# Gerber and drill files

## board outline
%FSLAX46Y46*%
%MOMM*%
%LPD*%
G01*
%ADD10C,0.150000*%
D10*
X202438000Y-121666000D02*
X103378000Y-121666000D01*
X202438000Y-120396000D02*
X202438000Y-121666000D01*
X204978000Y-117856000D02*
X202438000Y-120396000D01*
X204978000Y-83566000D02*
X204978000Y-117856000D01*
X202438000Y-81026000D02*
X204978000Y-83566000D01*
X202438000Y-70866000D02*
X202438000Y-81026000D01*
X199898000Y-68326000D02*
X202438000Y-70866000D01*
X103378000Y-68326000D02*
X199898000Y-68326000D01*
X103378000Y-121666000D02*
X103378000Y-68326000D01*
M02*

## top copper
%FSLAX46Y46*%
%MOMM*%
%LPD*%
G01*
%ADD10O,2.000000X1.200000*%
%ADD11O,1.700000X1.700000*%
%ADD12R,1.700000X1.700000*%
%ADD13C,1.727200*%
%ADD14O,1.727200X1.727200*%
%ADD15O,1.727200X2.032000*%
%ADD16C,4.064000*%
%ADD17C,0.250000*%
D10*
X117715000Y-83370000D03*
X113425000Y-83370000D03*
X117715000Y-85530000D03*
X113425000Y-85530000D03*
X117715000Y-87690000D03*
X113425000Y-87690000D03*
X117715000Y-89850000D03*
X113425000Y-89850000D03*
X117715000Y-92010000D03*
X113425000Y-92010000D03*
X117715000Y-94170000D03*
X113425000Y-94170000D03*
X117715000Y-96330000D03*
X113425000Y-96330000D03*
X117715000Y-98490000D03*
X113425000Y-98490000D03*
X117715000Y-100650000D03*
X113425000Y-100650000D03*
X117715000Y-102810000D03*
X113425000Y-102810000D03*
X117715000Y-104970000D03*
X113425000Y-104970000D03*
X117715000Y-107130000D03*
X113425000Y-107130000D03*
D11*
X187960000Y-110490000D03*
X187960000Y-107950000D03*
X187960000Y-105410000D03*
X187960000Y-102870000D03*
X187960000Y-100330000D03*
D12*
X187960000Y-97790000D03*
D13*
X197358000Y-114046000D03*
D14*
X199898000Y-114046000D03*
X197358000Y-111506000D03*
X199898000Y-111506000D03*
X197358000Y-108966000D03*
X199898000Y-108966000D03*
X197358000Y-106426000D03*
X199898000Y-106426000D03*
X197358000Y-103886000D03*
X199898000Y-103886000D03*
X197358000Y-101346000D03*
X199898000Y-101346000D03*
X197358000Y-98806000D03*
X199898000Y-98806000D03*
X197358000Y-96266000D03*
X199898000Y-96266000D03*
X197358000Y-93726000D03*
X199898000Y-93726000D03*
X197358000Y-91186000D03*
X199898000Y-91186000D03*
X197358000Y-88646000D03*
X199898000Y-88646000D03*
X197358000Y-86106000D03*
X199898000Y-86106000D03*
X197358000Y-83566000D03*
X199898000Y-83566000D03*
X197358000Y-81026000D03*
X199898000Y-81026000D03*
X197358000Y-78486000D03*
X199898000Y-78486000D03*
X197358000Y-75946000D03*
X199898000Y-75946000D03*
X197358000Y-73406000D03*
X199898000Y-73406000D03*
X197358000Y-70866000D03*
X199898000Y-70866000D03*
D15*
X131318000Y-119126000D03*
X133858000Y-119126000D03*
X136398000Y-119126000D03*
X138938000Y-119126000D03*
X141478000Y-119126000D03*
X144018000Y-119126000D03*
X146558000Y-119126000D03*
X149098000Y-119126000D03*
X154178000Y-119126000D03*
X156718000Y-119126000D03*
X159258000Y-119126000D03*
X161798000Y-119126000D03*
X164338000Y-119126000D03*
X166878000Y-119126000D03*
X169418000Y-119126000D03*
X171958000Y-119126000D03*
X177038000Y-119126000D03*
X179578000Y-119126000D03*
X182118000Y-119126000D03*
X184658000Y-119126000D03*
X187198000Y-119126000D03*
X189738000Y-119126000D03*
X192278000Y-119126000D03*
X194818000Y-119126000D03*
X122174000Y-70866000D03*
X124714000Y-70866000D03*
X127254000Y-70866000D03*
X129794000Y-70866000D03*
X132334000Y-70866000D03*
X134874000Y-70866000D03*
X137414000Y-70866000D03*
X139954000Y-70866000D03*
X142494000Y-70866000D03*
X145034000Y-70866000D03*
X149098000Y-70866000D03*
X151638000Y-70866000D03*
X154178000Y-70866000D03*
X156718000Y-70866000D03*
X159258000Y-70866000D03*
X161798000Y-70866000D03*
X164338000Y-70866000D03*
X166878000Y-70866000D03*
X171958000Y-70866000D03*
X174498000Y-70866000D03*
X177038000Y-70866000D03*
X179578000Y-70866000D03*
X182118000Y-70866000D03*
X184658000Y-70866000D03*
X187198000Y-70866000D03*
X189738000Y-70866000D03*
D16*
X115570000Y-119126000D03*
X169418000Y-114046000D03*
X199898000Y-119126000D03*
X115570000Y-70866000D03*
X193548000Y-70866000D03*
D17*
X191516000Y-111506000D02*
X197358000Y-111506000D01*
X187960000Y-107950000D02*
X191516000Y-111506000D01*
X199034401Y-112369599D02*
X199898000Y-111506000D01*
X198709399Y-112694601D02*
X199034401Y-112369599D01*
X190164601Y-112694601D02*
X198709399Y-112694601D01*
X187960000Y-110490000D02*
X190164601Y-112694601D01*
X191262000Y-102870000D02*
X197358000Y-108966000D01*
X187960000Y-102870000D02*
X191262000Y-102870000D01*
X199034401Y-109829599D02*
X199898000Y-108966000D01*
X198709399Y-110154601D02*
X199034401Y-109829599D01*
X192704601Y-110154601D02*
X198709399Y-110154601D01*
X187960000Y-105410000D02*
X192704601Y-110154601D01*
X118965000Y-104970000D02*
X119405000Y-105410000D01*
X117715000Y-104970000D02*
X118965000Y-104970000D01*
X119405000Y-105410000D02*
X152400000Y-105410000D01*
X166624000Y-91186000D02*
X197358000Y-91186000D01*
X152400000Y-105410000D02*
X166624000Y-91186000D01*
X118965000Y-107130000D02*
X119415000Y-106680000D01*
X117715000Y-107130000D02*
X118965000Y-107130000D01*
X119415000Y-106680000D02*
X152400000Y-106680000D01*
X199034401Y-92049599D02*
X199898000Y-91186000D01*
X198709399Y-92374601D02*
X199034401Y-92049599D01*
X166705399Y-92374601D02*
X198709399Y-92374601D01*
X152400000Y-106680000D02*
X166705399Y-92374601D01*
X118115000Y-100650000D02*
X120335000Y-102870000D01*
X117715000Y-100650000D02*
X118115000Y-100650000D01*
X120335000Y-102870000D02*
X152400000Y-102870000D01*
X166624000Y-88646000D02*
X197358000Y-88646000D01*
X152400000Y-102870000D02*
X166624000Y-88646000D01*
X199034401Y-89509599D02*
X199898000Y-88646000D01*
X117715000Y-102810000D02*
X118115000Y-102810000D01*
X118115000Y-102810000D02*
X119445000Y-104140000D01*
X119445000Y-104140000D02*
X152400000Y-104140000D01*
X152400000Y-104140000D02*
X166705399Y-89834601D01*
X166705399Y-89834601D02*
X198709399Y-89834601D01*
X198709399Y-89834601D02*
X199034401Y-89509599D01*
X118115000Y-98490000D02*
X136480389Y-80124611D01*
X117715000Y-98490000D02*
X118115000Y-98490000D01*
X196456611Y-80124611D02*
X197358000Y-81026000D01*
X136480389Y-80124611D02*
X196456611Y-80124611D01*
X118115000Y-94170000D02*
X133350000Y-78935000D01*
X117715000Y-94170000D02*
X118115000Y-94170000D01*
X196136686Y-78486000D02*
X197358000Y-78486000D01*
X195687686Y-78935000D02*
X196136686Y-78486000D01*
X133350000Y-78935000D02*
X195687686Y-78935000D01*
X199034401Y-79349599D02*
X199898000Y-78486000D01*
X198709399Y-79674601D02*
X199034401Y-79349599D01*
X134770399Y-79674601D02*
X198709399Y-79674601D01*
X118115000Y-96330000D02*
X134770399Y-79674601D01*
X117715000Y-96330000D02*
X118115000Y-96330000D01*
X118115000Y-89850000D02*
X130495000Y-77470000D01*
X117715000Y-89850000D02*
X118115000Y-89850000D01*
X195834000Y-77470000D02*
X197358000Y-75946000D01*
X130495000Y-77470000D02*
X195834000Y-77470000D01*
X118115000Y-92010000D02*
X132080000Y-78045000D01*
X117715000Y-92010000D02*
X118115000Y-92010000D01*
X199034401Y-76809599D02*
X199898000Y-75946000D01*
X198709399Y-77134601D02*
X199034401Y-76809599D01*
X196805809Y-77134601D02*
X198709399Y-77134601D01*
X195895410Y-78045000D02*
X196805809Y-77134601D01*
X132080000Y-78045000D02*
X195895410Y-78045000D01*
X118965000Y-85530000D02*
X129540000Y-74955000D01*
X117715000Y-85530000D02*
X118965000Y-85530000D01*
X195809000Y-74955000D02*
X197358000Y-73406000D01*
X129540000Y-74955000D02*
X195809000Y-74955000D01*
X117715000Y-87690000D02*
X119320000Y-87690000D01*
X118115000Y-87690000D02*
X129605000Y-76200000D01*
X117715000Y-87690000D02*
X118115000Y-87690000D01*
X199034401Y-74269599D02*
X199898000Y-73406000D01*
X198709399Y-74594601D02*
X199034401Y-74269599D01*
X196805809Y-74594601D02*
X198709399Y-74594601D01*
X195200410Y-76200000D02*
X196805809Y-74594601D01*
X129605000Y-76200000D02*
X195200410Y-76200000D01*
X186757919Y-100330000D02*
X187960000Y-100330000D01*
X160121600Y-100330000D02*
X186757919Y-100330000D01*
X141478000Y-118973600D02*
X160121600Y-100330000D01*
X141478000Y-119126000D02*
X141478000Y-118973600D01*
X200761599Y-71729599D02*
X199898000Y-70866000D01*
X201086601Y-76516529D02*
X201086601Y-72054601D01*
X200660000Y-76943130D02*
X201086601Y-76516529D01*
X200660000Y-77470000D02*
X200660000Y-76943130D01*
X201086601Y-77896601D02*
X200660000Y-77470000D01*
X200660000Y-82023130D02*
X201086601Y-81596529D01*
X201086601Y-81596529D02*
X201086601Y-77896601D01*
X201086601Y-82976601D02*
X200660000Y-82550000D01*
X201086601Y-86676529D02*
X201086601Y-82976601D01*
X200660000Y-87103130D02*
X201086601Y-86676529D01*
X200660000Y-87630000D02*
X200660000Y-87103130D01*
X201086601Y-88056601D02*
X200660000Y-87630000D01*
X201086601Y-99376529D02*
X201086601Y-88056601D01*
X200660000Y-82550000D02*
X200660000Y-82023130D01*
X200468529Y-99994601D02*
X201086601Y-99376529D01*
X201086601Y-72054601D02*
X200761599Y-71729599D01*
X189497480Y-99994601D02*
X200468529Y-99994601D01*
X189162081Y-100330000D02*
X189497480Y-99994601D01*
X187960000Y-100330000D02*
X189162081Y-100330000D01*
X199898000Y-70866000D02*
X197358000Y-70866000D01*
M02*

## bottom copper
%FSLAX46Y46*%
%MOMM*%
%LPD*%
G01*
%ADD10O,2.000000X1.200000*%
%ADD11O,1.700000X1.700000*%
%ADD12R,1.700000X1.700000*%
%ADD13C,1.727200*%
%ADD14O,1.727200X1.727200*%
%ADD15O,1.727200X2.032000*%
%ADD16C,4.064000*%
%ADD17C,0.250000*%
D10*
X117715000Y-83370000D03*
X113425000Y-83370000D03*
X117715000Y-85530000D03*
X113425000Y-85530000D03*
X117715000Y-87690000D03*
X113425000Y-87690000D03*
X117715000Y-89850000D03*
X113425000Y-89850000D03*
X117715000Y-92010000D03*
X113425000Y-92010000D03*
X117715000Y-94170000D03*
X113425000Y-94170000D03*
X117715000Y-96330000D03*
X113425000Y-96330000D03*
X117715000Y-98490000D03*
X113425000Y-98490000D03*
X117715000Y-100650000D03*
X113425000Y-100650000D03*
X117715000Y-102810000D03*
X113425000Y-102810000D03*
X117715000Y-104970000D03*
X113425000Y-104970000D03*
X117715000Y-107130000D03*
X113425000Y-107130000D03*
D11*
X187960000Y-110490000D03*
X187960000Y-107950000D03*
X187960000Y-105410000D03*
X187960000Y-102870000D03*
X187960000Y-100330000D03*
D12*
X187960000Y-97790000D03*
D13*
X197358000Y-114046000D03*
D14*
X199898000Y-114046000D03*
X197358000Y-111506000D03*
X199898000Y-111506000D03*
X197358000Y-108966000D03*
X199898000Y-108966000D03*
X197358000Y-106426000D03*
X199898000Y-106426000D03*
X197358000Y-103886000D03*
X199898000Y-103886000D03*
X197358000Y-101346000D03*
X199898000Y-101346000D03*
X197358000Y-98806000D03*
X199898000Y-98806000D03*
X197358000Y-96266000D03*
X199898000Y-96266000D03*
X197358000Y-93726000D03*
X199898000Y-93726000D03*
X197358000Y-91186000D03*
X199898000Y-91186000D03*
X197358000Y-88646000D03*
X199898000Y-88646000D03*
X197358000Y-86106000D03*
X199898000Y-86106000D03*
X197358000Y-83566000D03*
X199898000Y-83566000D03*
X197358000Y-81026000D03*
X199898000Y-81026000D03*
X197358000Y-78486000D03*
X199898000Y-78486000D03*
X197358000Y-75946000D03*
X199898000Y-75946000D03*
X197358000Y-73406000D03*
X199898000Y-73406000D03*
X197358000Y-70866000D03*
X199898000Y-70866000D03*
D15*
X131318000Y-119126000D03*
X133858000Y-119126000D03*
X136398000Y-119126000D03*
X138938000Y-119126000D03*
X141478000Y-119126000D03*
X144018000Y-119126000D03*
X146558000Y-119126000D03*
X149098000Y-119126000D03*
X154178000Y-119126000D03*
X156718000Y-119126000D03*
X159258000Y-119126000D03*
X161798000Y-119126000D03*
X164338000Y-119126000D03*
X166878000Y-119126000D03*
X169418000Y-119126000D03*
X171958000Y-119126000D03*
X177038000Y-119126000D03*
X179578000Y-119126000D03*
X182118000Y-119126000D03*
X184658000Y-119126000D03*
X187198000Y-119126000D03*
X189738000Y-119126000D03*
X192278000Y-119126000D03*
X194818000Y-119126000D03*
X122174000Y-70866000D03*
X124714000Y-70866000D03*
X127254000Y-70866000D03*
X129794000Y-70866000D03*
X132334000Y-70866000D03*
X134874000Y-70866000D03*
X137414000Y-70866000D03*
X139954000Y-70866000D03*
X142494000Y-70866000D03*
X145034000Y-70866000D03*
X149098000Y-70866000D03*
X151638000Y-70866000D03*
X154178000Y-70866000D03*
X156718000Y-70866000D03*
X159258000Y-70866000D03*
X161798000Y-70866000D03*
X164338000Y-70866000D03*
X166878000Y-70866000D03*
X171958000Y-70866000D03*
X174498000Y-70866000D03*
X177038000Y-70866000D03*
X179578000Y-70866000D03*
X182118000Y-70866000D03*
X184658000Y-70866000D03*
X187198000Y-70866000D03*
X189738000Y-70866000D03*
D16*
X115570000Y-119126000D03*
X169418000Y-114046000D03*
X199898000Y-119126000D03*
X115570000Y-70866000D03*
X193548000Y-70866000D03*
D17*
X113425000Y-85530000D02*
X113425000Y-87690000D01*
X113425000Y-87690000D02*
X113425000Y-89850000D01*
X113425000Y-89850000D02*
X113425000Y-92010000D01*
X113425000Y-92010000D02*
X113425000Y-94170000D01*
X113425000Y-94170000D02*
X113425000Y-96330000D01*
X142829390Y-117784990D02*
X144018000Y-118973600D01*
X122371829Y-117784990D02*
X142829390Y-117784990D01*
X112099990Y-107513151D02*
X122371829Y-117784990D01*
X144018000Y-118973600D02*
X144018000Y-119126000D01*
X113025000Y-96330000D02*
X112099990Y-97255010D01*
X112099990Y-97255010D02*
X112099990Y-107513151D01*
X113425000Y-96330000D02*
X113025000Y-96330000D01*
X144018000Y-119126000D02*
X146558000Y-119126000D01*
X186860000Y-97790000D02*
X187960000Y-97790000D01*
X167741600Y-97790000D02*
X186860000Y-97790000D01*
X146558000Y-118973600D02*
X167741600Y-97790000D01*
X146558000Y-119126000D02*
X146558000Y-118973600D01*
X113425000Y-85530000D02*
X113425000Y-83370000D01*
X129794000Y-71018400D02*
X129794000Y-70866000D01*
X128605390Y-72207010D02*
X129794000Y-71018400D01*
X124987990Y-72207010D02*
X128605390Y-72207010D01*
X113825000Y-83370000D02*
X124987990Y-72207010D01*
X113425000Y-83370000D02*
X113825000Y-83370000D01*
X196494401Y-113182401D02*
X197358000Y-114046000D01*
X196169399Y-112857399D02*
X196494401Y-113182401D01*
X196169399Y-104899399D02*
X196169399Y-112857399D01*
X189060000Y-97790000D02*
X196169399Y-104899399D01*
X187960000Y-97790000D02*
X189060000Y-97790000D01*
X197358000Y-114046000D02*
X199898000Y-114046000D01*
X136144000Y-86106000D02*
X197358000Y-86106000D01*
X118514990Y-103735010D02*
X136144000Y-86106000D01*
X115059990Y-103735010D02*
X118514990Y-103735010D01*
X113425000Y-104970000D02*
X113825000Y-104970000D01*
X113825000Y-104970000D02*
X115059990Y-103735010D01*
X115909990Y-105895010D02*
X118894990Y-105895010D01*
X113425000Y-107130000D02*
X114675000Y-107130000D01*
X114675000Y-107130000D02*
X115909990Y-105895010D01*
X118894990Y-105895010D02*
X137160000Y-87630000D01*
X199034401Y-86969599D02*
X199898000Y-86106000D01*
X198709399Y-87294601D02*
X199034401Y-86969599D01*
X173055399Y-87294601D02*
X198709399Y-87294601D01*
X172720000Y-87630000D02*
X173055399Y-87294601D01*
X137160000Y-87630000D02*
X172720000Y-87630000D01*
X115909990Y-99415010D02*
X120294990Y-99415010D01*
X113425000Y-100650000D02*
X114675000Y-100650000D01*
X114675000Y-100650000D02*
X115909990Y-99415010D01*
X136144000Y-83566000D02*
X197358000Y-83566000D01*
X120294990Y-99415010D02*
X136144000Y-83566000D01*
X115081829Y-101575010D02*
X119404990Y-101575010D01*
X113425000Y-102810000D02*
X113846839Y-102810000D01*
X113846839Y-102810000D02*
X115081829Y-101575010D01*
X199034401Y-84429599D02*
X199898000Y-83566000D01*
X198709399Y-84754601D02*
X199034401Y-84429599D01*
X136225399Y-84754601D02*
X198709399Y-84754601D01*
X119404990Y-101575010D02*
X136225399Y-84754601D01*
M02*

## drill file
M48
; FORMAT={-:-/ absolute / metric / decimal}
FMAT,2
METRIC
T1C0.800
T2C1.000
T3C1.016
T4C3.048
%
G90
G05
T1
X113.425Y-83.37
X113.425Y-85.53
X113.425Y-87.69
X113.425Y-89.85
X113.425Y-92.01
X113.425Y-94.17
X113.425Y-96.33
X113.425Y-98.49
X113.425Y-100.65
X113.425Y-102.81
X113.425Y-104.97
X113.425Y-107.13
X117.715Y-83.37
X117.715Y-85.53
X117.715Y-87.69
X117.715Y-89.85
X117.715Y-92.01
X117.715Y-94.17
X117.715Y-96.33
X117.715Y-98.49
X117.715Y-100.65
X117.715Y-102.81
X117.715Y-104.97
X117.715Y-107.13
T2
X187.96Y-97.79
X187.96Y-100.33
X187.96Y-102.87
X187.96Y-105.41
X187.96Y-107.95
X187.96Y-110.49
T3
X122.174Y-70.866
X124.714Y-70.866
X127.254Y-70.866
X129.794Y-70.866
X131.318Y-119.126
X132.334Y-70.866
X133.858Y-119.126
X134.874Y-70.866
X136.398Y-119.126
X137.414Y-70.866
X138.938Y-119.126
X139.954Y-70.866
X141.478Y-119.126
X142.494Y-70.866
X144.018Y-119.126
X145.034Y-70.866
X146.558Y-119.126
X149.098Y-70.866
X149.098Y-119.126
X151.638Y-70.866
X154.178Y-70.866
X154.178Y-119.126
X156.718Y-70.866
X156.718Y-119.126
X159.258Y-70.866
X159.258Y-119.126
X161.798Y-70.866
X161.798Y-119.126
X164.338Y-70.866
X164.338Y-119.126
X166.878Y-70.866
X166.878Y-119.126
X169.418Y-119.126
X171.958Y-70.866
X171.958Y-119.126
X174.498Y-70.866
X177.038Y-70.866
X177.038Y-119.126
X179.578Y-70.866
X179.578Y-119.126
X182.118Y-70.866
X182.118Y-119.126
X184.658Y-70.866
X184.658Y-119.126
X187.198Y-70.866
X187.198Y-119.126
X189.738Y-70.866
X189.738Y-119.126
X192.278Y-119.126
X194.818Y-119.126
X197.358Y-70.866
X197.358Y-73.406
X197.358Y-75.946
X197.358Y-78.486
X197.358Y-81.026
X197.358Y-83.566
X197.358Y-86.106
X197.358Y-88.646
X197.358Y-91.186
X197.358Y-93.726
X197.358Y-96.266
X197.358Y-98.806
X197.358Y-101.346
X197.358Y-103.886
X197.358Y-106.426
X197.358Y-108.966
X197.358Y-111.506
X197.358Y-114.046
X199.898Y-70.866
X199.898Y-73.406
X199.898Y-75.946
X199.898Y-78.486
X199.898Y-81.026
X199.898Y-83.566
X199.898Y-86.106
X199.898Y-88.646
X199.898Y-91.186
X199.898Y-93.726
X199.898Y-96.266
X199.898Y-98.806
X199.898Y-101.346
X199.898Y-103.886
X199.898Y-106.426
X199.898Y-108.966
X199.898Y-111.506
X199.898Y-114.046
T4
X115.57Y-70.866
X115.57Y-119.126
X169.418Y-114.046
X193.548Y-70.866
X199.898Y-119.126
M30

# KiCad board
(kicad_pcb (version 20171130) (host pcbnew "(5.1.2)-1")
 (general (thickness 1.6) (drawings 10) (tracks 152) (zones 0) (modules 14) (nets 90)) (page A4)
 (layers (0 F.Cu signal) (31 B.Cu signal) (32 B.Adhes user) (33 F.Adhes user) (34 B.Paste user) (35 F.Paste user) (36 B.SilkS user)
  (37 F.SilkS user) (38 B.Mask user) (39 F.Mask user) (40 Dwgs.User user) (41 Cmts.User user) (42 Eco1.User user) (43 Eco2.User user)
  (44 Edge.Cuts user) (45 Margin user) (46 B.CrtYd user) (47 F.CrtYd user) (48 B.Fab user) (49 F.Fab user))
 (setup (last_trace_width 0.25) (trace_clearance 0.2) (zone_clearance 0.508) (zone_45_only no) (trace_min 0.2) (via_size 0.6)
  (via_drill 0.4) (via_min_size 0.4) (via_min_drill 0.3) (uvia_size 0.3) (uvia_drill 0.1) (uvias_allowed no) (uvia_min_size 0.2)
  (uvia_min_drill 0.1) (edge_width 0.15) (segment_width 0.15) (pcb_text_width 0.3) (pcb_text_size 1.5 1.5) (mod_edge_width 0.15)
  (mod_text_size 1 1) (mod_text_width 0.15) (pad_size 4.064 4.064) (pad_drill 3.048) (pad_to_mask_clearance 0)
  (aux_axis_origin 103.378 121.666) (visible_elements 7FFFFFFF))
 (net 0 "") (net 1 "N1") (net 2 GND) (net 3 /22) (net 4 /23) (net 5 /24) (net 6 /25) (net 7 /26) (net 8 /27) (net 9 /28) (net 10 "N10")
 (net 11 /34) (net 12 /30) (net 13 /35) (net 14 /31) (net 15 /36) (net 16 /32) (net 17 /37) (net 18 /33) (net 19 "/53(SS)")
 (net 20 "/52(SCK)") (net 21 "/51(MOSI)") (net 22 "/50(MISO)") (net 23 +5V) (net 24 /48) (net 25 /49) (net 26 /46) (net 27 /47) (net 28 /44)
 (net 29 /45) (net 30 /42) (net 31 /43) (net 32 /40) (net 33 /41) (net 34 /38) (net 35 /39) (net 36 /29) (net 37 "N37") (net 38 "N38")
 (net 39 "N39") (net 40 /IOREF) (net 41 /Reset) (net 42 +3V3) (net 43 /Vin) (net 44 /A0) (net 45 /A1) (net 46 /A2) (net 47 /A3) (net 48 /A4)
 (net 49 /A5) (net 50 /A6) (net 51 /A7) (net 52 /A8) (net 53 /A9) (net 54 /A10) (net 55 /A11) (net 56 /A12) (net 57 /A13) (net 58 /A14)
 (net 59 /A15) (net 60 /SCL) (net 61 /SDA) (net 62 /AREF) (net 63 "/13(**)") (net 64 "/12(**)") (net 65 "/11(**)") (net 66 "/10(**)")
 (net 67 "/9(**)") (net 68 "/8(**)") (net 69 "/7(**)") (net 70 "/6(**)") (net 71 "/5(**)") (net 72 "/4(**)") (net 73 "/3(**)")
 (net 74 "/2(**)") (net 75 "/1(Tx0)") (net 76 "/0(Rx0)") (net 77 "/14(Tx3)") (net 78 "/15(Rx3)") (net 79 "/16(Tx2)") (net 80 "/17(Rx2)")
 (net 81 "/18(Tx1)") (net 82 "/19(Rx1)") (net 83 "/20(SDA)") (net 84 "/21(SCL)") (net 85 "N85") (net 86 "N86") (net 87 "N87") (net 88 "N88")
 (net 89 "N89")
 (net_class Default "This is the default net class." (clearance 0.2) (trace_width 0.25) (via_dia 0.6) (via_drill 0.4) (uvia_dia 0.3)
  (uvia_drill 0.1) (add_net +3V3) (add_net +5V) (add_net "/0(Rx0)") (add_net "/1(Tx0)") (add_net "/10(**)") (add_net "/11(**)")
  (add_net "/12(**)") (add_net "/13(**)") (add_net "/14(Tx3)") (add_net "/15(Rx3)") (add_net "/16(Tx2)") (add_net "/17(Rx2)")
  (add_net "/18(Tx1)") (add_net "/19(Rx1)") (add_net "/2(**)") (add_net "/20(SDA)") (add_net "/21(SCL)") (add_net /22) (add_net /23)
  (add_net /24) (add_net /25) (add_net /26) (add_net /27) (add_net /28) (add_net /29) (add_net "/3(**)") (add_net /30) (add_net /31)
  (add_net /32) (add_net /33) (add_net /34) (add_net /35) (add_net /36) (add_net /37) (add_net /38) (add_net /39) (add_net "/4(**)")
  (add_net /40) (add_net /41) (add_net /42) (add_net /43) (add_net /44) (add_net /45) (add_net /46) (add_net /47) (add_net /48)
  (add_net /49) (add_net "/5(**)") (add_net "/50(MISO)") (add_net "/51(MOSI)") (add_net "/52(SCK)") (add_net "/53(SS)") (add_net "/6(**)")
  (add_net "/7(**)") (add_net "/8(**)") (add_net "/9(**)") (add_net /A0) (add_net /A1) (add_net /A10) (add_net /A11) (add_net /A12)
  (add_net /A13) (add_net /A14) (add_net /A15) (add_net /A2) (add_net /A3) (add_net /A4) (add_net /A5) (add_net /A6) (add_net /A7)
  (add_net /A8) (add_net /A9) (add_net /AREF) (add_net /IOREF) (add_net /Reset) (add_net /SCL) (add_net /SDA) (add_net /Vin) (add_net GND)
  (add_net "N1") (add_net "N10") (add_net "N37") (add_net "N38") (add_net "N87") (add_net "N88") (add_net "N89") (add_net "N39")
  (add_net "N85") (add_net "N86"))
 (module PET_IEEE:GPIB (layer F.Cu) (at 115.57 95.25 90)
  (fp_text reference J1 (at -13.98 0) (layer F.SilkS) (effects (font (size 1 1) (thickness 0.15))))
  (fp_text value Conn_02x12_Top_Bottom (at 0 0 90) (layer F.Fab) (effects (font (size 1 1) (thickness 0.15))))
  (pad 12 thru_hole oval (at 11.88 2.145 90) (size 1.2 2) (drill 0.8) (layers *.Cu *.Mask) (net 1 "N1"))
  (pad 24 thru_hole oval (at 11.88 -2.145 90) (size 1.2 2) (drill 0.8) (layers *.Cu *.Mask) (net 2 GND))
  (pad 11 thru_hole oval (at 9.72 2.145 90) (size 1.2 2) (drill 0.8) (layers *.Cu *.Mask) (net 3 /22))
  (pad 23 thru_hole oval (at 9.72 -2.145 90) (size 1.2 2) (drill 0.8) (layers *.Cu *.Mask) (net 2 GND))
  (pad 10 thru_hole oval (at 7.56 2.145 90) (size 1.2 2) (drill 0.8) (layers *.Cu *.Mask) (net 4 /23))
  (pad 22 thru_hole oval (at 7.56 -2.145 90) (size 1.2 2) (drill 0.8) (layers *.Cu *.Mask) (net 2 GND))
  (pad 9 thru_hole oval (at 5.4 2.145 90) (size 1.2 2) (drill 0.8) (layers *.Cu *.Mask) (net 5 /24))
  (pad 21 thru_hole oval (at 5.4 -2.145 90) (size 1.2 2) (drill 0.8) (layers *.Cu *.Mask) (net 2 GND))
  (pad 8 thru_hole oval (at 3.24 2.145 90) (size 1.2 2) (drill 0.8) (layers *.Cu *.Mask) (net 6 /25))
  (pad 20 thru_hole oval (at 3.24 -2.145 90) (size 1.2 2) (drill 0.8) (layers *.Cu *.Mask) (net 2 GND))
  (pad 7 thru_hole oval (at 1.08 2.145 90) (size 1.2 2) (drill 0.8) (layers *.Cu *.Mask) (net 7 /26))
  (pad 19 thru_hole oval (at 1.08 -2.145 90) (size 1.2 2) (drill 0.8) (layers *.Cu *.Mask) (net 2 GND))
  (pad 6 thru_hole oval (at -1.08 2.145 90) (size 1.2 2) (drill 0.8) (layers *.Cu *.Mask) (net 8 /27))
  (pad 18 thru_hole oval (at -1.08 -2.145 90) (size 1.2 2) (drill 0.8) (layers *.Cu *.Mask) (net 2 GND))
  (pad 5 thru_hole oval (at -3.24 2.145 90) (size 1.2 2) (drill 0.8) (layers *.Cu *.Mask) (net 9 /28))
  (pad 17 thru_hole oval (at -3.24 -2.145 90) (size 1.2 2) (drill 0.8) (layers *.Cu *.Mask) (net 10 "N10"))
  (pad 4 thru_hole oval (at -5.4 2.145 90) (size 1.2 2) (drill 0.8) (layers *.Cu *.Mask) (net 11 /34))
  (pad 16 thru_hole oval (at -5.4 -2.145 90) (size 1.2 2) (drill 0.8) (layers *.Cu *.Mask) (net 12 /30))
  (pad 3 thru_hole oval (at -7.56 2.145 90) (size 1.2 2) (drill 0.8) (layers *.Cu *.Mask) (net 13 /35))
  (pad 15 thru_hole oval (at -7.56 -2.145 90) (size 1.2 2) (drill 0.8) (layers *.Cu *.Mask) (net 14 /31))
  (pad 2 thru_hole oval (at -9.72 2.145 90) (size 1.2 2) (drill 0.8) (layers *.Cu *.Mask) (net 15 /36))
  (pad 14 thru_hole oval (at -9.72 -2.145 90) (size 1.2 2) (drill 0.8) (layers *.Cu *.Mask) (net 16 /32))
  (pad 1 thru_hole oval (at -11.88 2.145 90) (size 1.2 2) (drill 0.8) (layers *.Cu *.Mask) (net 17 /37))
  (pad 13 thru_hole oval (at -11.88 -2.145 90) (size 1.2 2) (drill 0.8) (layers *.Cu *.Mask) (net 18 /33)))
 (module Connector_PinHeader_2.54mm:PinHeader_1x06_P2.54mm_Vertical (layer F.Cu) (at 187.96 97.79)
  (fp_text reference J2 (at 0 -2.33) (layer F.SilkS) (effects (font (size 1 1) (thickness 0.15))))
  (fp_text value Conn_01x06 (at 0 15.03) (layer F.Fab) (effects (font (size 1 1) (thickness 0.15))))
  (pad 6 thru_hole oval (at 0 12.7) (size 1.7 1.7) (drill 1) (layers *.Cu *.Mask) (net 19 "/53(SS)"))
  (pad 5 thru_hole oval (at 0 10.16) (size 1.7 1.7) (drill 1) (layers *.Cu *.Mask) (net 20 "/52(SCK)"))
  (pad 4 thru_hole oval (at 0 7.62) (size 1.7 1.7) (drill 1) (layers *.Cu *.Mask) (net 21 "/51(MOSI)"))
  (pad 3 thru_hole oval (at 0 5.08) (size 1.7 1.7) (drill 1) (layers *.Cu *.Mask) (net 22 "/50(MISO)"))
  (pad 2 thru_hole oval (at 0 2.54) (size 1.7 1.7) (drill 1) (layers *.Cu *.Mask) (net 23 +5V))
  (pad 1 thru_hole rect (at 0 0) (size 1.7 1.7) (drill 1) (layers *.Cu *.Mask) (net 2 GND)))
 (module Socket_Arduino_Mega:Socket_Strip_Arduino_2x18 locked (layer F.Cu) (at 197.358 114.046 90)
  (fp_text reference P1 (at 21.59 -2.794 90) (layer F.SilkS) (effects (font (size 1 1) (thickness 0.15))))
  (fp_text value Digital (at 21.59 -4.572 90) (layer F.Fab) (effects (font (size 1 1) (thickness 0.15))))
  (pad 1 thru_hole circle (at 0 0 90) (size 1.7272 1.7272) (drill 1.016) (layers *.Cu *.Mask F.SilkS) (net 2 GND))
  (pad 2 thru_hole oval (at 0 2.54 90) (size 1.7272 1.7272) (drill 1.016) (layers *.Cu *.Mask F.SilkS) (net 2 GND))
  (pad 3 thru_hole oval (at 2.54 0 90) (size 1.7272 1.7272) (drill 1.016) (layers *.Cu *.Mask F.SilkS) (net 20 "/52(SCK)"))
  (pad 4 thru_hole oval (at 2.54 2.54 90) (size 1.7272 1.7272) (drill 1.016) (layers *.Cu *.Mask F.SilkS) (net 19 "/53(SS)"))
  (pad 5 thru_hole oval (at 5.08 0 90) (size 1.7272 1.7272) (drill 1.016) (layers *.Cu *.Mask F.SilkS) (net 22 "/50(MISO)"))
  (pad 6 thru_hole oval (at 5.08 2.54 90) (size 1.7272 1.7272) (drill 1.016) (layers *.Cu *.Mask F.SilkS) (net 21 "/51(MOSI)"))
  (pad 7 thru_hole oval (at 7.62 0 90) (size 1.7272 1.7272) (drill 1.016) (layers *.Cu *.Mask F.SilkS) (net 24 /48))
  (pad 8 thru_hole oval (at 7.62 2.54 90) (size 1.7272 1.7272) (drill 1.016) (layers *.Cu *.Mask F.SilkS) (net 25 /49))
  (pad 9 thru_hole oval (at 10.16 0 90) (size 1.7272 1.7272) (drill 1.016) (layers *.Cu *.Mask F.SilkS) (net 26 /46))
  (pad 10 thru_hole oval (at 10.16 2.54 90) (size 1.7272 1.7272) (drill 1.016) (layers *.Cu *.Mask F.SilkS) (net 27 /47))
  (pad 11 thru_hole oval (at 12.7 0 90) (size 1.7272 1.7272) (drill 1.016) (layers *.Cu *.Mask F.SilkS) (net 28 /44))
  (pad 12 thru_hole oval (at 12.7 2.54 90) (size 1.7272 1.7272) (drill 1.016) (layers *.Cu *.Mask F.SilkS) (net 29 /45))
  (pad 13 thru_hole oval (at 15.24 0 90) (size 1.7272 1.7272) (drill 1.016) (layers *.Cu *.Mask F.SilkS) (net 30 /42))
  (pad 14 thru_hole oval (at 15.24 2.54 90) (size 1.7272 1.7272) (drill 1.016) (layers *.Cu *.Mask F.SilkS) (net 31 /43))
  (pad 15 thru_hole oval (at 17.78 0 90) (size 1.7272 1.7272) (drill 1.016) (layers *.Cu *.Mask F.SilkS) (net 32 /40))
  (pad 16 thru_hole oval (at 17.78 2.54 90) (size 1.7272 1.7272) (drill 1.016) (layers *.Cu *.Mask F.SilkS) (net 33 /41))
  (pad 17 thru_hole oval (at 20.32 0 90) (size 1.7272 1.7272) (drill 1.016) (layers *.Cu *.Mask F.SilkS) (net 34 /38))
  (pad 18 thru_hole oval (at 20.32 2.54 90) (size 1.7272 1.7272) (drill 1.016) (layers *.Cu *.Mask F.SilkS) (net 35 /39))
  (pad 19 thru_hole oval (at 22.86 0 90) (size 1.7272 1.7272) (drill 1.016) (layers *.Cu *.Mask F.SilkS) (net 15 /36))
  (pad 20 thru_hole oval (at 22.86 2.54 90) (size 1.7272 1.7272) (drill 1.016) (layers *.Cu *.Mask F.SilkS) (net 17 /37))
  (pad 21 thru_hole oval (at 25.4 0 90) (size 1.7272 1.7272) (drill 1.016) (layers *.Cu *.Mask F.SilkS) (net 11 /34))
  (pad 22 thru_hole oval (at 25.4 2.54 90) (size 1.7272 1.7272) (drill 1.016) (layers *.Cu *.Mask F.SilkS) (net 13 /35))
  (pad 23 thru_hole oval (at 27.94 0 90) (size 1.7272 1.7272) (drill 1.016) (layers *.Cu *.Mask F.SilkS) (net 16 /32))
  (pad 24 thru_hole oval (at 27.94 2.54 90) (size 1.7272 1.7272) (drill 1.016) (layers *.Cu *.Mask F.SilkS) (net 18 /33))
  (pad 25 thru_hole oval (at 30.48 0 90) (size 1.7272 1.7272) (drill 1.016) (layers *.Cu *.Mask F.SilkS) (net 12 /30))
  (pad 26 thru_hole oval (at 30.48 2.54 90) (size 1.7272 1.7272) (drill 1.016) (layers *.Cu *.Mask F.SilkS) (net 14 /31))
  (pad 27 thru_hole oval (at 33.02 0 90) (size 1.7272 1.7272) (drill 1.016) (layers *.Cu *.Mask F.SilkS) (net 9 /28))
  (pad 28 thru_hole oval (at 33.02 2.54 90) (size 1.7272 1.7272) (drill 1.016) (layers *.Cu *.Mask F.SilkS) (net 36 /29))
  (pad 29 thru_hole oval (at 35.56 0 90) (size 1.7272 1.7272) (drill 1.016) (layers *.Cu *.Mask F.SilkS) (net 7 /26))
  (pad 30 thru_hole oval (at 35.56 2.54 90) (size 1.7272 1.7272) (drill 1.016) (layers *.Cu *.Mask F.SilkS) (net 8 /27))
  (pad 31 thru_hole oval (at 38.1 0 90) (size 1.7272 1.7272) (drill 1.016) (layers *.Cu *.Mask F.SilkS) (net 5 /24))
  (pad 32 thru_hole oval (at 38.1 2.54 90) (size 1.7272 1.7272) (drill 1.016) (layers *.Cu *.Mask F.SilkS) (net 6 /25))
  (pad 33 thru_hole oval (at 40.64 0 90) (size 1.7272 1.7272) (drill 1.016) (layers *.Cu *.Mask F.SilkS) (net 3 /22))
  (pad 34 thru_hole oval (at 40.64 2.54 90) (size 1.7272 1.7272) (drill 1.016) (layers *.Cu *.Mask F.SilkS) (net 4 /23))
  (pad 35 thru_hole oval (at 43.18 0 90) (size 1.7272 1.7272) (drill 1.016) (layers *.Cu *.Mask F.SilkS) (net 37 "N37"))
  (pad 36 thru_hole oval (at 43.18 2.54 90) (size 1.7272 1.7272) (drill 1.016) (layers *.Cu *.Mask F.SilkS) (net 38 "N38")))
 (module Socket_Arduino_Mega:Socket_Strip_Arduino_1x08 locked (layer F.Cu) (at 131.318 119.126)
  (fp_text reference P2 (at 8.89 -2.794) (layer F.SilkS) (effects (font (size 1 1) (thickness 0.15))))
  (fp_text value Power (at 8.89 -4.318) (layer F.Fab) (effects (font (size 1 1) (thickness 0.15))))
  (pad 1 thru_hole oval (at 0 0) (size 1.7272 2.032) (drill 1.016) (layers *.Cu *.Mask F.SilkS) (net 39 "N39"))
  (pad 2 thru_hole oval (at 2.54 0) (size 1.7272 2.032) (drill 1.016) (layers *.Cu *.Mask F.SilkS) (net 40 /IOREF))
  (pad 3 thru_hole oval (at 5.08 0) (size 1.7272 2.032) (drill 1.016) (layers *.Cu *.Mask F.SilkS) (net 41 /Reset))
  (pad 4 thru_hole oval (at 7.62 0) (size 1.7272 2.032) (drill 1.016) (layers *.Cu *.Mask F.SilkS) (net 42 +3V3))
  (pad 5 thru_hole oval (at 10.16 0) (size 1.7272 2.032) (drill 1.016) (layers *.Cu *.Mask F.SilkS) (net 23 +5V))
  (pad 6 thru_hole oval (at 12.7 0) (size 1.7272 2.032) (drill 1.016) (layers *.Cu *.Mask F.SilkS) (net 2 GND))
  (pad 7 thru_hole oval (at 15.24 0) (size 1.7272 2.032) (drill 1.016) (layers *.Cu *.Mask F.SilkS) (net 2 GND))
  (pad 8 thru_hole oval (at 17.78 0) (size 1.7272 2.032) (drill 1.016) (layers *.Cu *.Mask F.SilkS) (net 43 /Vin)))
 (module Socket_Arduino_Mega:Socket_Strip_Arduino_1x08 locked (layer F.Cu) (at 154.178 119.126)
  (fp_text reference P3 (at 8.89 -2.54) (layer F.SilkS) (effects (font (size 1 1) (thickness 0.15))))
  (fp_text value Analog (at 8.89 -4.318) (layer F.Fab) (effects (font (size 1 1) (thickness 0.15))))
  (pad 1 thru_hole oval (at 0 0) (size 1.7272 2.032) (drill 1.016) (layers *.Cu *.Mask F.SilkS) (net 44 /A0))
  (pad 2 thru_hole oval (at 2.54 0) (size 1.7272 2.032) (drill 1.016) (layers *.Cu *.Mask F.SilkS) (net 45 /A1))
  (pad 3 thru_hole oval (at 5.08 0) (size 1.7272 2.032) (drill 1.016) (layers *.Cu *.Mask F.SilkS) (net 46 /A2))
  (pad 4 thru_hole oval (at 7.62 0) (size 1.7272 2.032) (drill 1.016) (layers *.Cu *.Mask F.SilkS) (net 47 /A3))
  (pad 5 thru_hole oval (at 10.16 0) (size 1.7272 2.032) (drill 1.016) (layers *.Cu *.Mask F.SilkS) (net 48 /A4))
  (pad 6 thru_hole oval (at 12.7 0) (size 1.7272 2.032) (drill 1.016) (layers *.Cu *.Mask F.SilkS) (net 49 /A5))
  (pad 7 thru_hole oval (at 15.24 0) (size 1.7272 2.032) (drill 1.016) (layers *.Cu *.Mask F.SilkS) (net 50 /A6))
  (pad 8 thru_hole oval (at 17.78 0) (size 1.7272 2.032) (drill 1.016) (layers *.Cu *.Mask F.SilkS) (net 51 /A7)))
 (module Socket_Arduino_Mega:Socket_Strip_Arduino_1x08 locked (layer F.Cu) (at 177.038 119.126)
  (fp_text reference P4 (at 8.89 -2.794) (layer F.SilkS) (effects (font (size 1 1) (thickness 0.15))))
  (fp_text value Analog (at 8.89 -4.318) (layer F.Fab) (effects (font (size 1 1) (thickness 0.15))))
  (pad 1 thru_hole oval (at 0 0) (size 1.7272 2.032) (drill 1.016) (layers *.Cu *.Mask F.SilkS) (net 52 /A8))
  (pad 2 thru_hole oval (at 2.54 0) (size 1.7272 2.032) (drill 1.016) (layers *.Cu *.Mask F.SilkS) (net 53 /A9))
  (pad 3 thru_hole oval (at 5.08 0) (size 1.7272 2.032) (drill 1.016) (layers *.Cu *.Mask F.SilkS) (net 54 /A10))
  (pad 4 thru_hole oval (at 7.62 0) (size 1.7272 2.032) (drill 1.016) (layers *.Cu *.Mask F.SilkS) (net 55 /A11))
  (pad 5 thru_hole oval (at 10.16 0) (size 1.7272 2.032) (drill 1.016) (layers *.Cu *.Mask F.SilkS) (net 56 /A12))
  (pad 6 thru_hole oval (at 12.7 0) (size 1.7272 2.032) (drill 1.016) (layers *.Cu *.Mask F.SilkS) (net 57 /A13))
  (pad 7 thru_hole oval (at 15.24 0) (size 1.7272 2.032) (drill 1.016) (layers *.Cu *.Mask F.SilkS) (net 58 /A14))
  (pad 8 thru_hole oval (at 17.78 0) (size 1.7272 2.032) (drill 1.016) (layers *.Cu *.Mask F.SilkS) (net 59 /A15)))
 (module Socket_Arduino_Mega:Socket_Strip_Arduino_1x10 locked (layer F.Cu) (at 122.174 70.866)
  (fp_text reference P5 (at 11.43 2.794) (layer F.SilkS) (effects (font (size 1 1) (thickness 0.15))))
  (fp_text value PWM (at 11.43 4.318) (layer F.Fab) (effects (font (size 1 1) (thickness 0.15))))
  (pad 1 thru_hole oval (at 0 0) (size 1.7272 2.032) (drill 1.016) (layers *.Cu *.Mask F.SilkS) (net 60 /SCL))
  (pad 2 thru_hole oval (at 2.54 0) (size 1.7272 2.032) (drill 1.016) (layers *.Cu *.Mask F.SilkS) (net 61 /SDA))
  (pad 3 thru_hole oval (at 5.08 0) (size 1.7272 2.032) (drill 1.016) (layers *.Cu *.Mask F.SilkS) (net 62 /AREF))
  (pad 4 thru_hole oval (at 7.62 0) (size 1.7272 2.032) (drill 1.016) (layers *.Cu *.Mask F.SilkS) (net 2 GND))
  (pad 5 thru_hole oval (at 10.16 0) (size 1.7272 2.032) (drill 1.016) (layers *.Cu *.Mask F.SilkS) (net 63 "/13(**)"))
  (pad 6 thru_hole oval (at 12.7 0) (size 1.7272 2.032) (drill 1.016) (layers *.Cu *.Mask F.SilkS) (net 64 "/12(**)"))
  (pad 7 thru_hole oval (at 15.24 0) (size 1.7272 2.032) (drill 1.016) (layers *.Cu *.Mask F.SilkS) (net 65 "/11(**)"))
  (pad 8 thru_hole oval (at 17.78 0) (size 1.7272 2.032) (drill 1.016) (layers *.Cu *.Mask F.SilkS) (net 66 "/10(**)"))
  (pad 9 thru_hole oval (at 20.32 0) (size 1.7272 2.032) (drill 1.016) (layers *.Cu *.Mask F.SilkS) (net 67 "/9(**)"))
  (pad 10 thru_hole oval (at 22.86 0) (size 1.7272 2.032) (drill 1.016) (layers *.Cu *.Mask F.SilkS) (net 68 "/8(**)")))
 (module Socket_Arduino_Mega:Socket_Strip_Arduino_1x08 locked (layer F.Cu) (at 149.098 70.866)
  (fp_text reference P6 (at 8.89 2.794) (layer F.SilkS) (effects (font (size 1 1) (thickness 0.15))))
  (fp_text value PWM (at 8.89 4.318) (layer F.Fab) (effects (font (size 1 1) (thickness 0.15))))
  (pad 1 thru_hole oval (at 0 0) (size 1.7272 2.032) (drill 1.016) (layers *.Cu *.Mask F.SilkS) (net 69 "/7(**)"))
  (pad 2 thru_hole oval (at 2.54 0) (size 1.7272 2.032) (drill 1.016) (layers *.Cu *.Mask F.SilkS) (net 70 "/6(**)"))
  (pad 3 thru_hole oval (at 5.08 0) (size 1.7272 2.032) (drill 1.016) (layers *.Cu *.Mask F.SilkS) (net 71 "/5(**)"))
  (pad 4 thru_hole oval (at 7.62 0) (size 1.7272 2.032) (drill 1.016) (layers *.Cu *.Mask F.SilkS) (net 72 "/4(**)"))
  (pad 5 thru_hole oval (at 10.16 0) (size 1.7272 2.032) (drill 1.016) (layers *.Cu *.Mask F.SilkS) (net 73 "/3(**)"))
  (pad 6 thru_hole oval (at 12.7 0) (size 1.7272 2.032) (drill 1.016) (layers *.Cu *.Mask F.SilkS) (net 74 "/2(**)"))
  (pad 7 thru_hole oval (at 15.24 0) (size 1.7272 2.032) (drill 1.016) (layers *.Cu *.Mask F.SilkS) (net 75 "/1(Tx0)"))
  (pad 8 thru_hole oval (at 17.78 0) (size 1.7272 2.032) (drill 1.016) (layers *.Cu *.Mask F.SilkS) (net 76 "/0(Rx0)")))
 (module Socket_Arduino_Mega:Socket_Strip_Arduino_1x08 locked (layer F.Cu) (at 171.958 70.866)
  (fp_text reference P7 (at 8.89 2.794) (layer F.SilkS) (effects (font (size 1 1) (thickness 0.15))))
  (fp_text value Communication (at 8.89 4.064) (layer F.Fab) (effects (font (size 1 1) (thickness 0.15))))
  (pad 1 thru_hole oval (at 0 0) (size 1.7272 2.032) (drill 1.016) (layers *.Cu *.Mask F.SilkS) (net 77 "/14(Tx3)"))
  (pad 2 thru_hole oval (at 2.54 0) (size 1.7272 2.032) (drill 1.016) (layers *.Cu *.Mask F.SilkS) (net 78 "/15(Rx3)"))
  (pad 3 thru_hole oval (at 5.08 0) (size 1.7272 2.032) (drill 1.016) (layers *.Cu *.Mask F.SilkS) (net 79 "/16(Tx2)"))
  (pad 4 thru_hole oval (at 7.62 0) (size 1.7272 2.032) (drill 1.016) (layers *.Cu *.Mask F.SilkS) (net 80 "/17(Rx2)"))
  (pad 5 thru_hole oval (at 10.16 0) (size 1.7272 2.032) (drill 1.016) (layers *.Cu *.Mask F.SilkS) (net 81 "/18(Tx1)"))
  (pad 6 thru_hole oval (at 12.7 0) (size 1.7272 2.032) (drill 1.016) (layers *.Cu *.Mask F.SilkS) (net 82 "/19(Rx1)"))
  (pad 7 thru_hole oval (at 15.24 0) (size 1.7272 2.032) (drill 1.016) (layers *.Cu *.Mask F.SilkS) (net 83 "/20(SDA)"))
  (pad 8 thru_hole oval (at 17.78 0) (size 1.7272 2.032) (drill 1.016) (layers *.Cu *.Mask F.SilkS) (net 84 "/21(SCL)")))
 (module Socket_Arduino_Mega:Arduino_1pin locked (layer F.Cu) (at 115.57 119.126)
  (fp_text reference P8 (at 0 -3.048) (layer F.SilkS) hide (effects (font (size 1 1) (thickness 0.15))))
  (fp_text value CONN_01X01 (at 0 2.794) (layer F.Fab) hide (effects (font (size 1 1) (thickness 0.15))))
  (pad 1 thru_hole circle (at 0 0) (size 4.064 4.064) (drill 3.048) (layers *.Cu *.Mask F.SilkS) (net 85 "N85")))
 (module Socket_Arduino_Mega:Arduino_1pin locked (layer F.Cu) (at 169.418 114.046)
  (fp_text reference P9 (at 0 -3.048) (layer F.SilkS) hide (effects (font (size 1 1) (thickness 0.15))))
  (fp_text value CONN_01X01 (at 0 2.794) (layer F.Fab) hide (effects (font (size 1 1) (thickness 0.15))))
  (pad 1 thru_hole circle (at 0 0) (size 4.064 4.064) (drill 3.048) (layers *.Cu *.Mask F.SilkS) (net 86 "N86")))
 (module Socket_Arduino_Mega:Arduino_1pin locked (layer F.Cu) (at 199.898 119.126)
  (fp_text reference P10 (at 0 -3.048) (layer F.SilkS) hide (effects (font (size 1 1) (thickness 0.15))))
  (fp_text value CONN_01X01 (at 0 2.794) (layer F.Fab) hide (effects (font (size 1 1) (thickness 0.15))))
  (pad 1 thru_hole circle (at 0 0) (size 4.064 4.064) (drill 3.048) (layers *.Cu *.Mask F.SilkS) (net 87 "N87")))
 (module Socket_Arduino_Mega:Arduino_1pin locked (layer F.Cu) (at 115.57 70.866)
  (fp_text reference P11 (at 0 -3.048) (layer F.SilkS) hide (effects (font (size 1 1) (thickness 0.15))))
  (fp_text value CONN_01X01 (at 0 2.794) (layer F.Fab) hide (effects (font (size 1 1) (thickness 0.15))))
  (pad 1 thru_hole circle (at 0 0) (size 4.064 4.064) (drill 3.048) (layers *.Cu *.Mask F.SilkS) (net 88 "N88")))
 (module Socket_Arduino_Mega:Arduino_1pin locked (layer F.Cu) (at 193.548 70.866)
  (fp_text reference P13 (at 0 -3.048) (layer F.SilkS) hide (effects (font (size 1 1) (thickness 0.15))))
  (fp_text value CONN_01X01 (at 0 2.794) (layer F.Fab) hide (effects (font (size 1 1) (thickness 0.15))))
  (pad 1 thru_hole circle (at 0 0) (size 4.064 4.064) (drill 3.048) (layers *.Cu *.Mask F.SilkS) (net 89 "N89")))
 (gr_line (start 202.438 121.666) (end 103.378 121.666) (angle 90) (layer Edge.Cuts) (width 0.15))
 (gr_line (start 202.438 120.396) (end 202.438 121.666) (angle 90) (layer Edge.Cuts) (width 0.15))
 (gr_line (start 204.978 117.856) (end 202.438 120.396) (angle 90) (layer Edge.Cuts) (width 0.15))
 (gr_line (start 204.978 83.566) (end 204.978 117.856) (angle 90) (layer Edge.Cuts) (width 0.15))
 (gr_line (start 202.438 81.026) (end 204.978 83.566) (angle 90) (layer Edge.Cuts) (width 0.15))
 (gr_line (start 202.438 70.866) (end 202.438 81.026) (angle 90) (layer Edge.Cuts) (width 0.15))
 (gr_line (start 199.898 68.326) (end 202.438 70.866) (angle 90) (layer Edge.Cuts) (width 0.15))
 (gr_line (start 103.378 68.326) (end 199.898 68.326) (angle 90) (layer Edge.Cuts) (width 0.15))
 (gr_line (start 103.378 121.666) (end 103.378 68.326) (angle 90) (layer Edge.Cuts) (width 0.15))
 (segment (start 113.425 85.53) (end 113.425 87.69) (width 0.25) (layer B.Cu) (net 2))
 (segment (start 113.425 87.69) (end 113.425 89.85) (width 0.25) (layer B.Cu) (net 2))
 (segment (start 113.425 89.85) (end 113.425 92.01) (width 0.25) (layer B.Cu) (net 2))
 (segment (start 113.425 92.01) (end 113.425 94.17) (width 0.25) (layer B.Cu) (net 2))
 (segment (start 113.425 94.17) (end 113.425 96.33) (width 0.25) (layer B.Cu) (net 2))
 (segment (start 142.82939 117.78499) (end 144.018 118.9736) (width 0.25) (layer B.Cu) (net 2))
 (segment (start 122.371829 117.78499) (end 142.82939 117.78499) (width 0.25) (layer B.Cu) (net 2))
 (segment (start 112.09999 107.513151) (end 122.371829 117.78499) (width 0.25) (layer B.Cu) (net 2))
 (segment (start 144.018 118.9736) (end 144.018 119.126) (width 0.25) (layer B.Cu) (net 2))
 (segment (start 113.025 96.33) (end 112.09999 97.25501) (width 0.25) (layer B.Cu) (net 2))
 (segment (start 112.09999 97.25501) (end 112.09999 107.513151) (width 0.25) (layer B.Cu) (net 2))
 (segment (start 113.425 96.33) (end 113.025 96.33) (width 0.25) (layer B.Cu) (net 2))
 (segment (start 144.018 119.126) (end 146.558 119.126) (width 0.25) (layer B.Cu) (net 2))
 (segment (start 186.86 97.79) (end 187.96 97.79) (width 0.25) (layer B.Cu) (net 2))
 (segment (start 167.7416 97.79) (end 186.86 97.79) (width 0.25) (layer B.Cu) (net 2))
 (segment (start 146.558 118.9736) (end 167.7416 97.79) (width 0.25) (layer B.Cu) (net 2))
 (segment (start 146.558 119.126) (end 146.558 118.9736) (width 0.25) (layer B.Cu) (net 2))
 (segment (start 113.425 85.53) (end 113.425 83.37) (width 0.25) (layer B.Cu) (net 2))
 (segment (start 129.794 71.0184) (end 129.794 70.866) (width 0.25) (layer B.Cu) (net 2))
 (segment (start 128.60539 72.20701) (end 129.794 71.0184) (width 0.25) (layer B.Cu) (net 2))
 (segment (start 124.98799 72.20701) (end 128.60539 72.20701) (width 0.25) (layer B.Cu) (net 2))
 (segment (start 113.825 83.37) (end 124.98799 72.20701) (width 0.25) (layer B.Cu) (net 2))
 (segment (start 113.425 83.37) (end 113.825 83.37) (width 0.25) (layer B.Cu) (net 2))
 (segment (start 196.494401 113.182401) (end 197.358 114.046) (width 0.25) (layer B.Cu) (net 2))
 (segment (start 196.169399 112.857399) (end 196.494401 113.182401) (width 0.25) (layer B.Cu) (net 2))
 (segment (start 196.169399 104.899399) (end 196.169399 112.857399) (width 0.25) (layer B.Cu) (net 2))
 (segment (start 189.06 97.79) (end 196.169399 104.899399) (width 0.25) (layer B.Cu) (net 2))
 (segment (start 187.96 97.79) (end 189.06 97.79) (width 0.25) (layer B.Cu) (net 2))
 (segment (start 197.358 114.046) (end 199.898 114.046) (width 0.25) (layer B.Cu) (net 2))
 (segment (start 191.516 111.506) (end 197.358 111.506) (width 0.25) (layer F.Cu) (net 20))
 (segment (start 187.96 107.95) (end 191.516 111.506) (width 0.25) (layer F.Cu) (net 20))
 (segment (start 199.034401 112.369599) (end 199.898 111.506) (width 0.25) (layer F.Cu) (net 19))
 (segment (start 198.709399 112.694601) (end 199.034401 112.369599) (width 0.25) (layer F.Cu) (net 19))
 (segment (start 190.164601 112.694601) (end 198.709399 112.694601) (width 0.25) (layer F.Cu) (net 19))
 (segment (start 187.96 110.49) (end 190.164601 112.694601) (width 0.25) (layer F.Cu) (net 19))
 (segment (start 191.262 102.87) (end 197.358 108.966) (width 0.25) (layer F.Cu) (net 22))
 (segment (start 187.96 102.87) (end 191.262 102.87) (width 0.25) (layer F.Cu) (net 22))
 (segment (start 199.034401 109.829599) (end 199.898 108.966) (width 0.25) (layer F.Cu) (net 21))
 (segment (start 198.709399 110.154601) (end 199.034401 109.829599) (width 0.25) (layer F.Cu) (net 21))
 (segment (start 192.704601 110.154601) (end 198.709399 110.154601) (width 0.25) (layer F.Cu) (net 21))
 (segment (start 187.96 105.41) (end 192.704601 110.154601) (width 0.25) (layer F.Cu) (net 21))
 (segment (start 118.965 104.97) (end 119.405 105.41) (width 0.25) (layer F.Cu) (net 15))
 (segment (start 117.715 104.97) (end 118.965 104.97) (width 0.25) (layer F.Cu) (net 15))
 (segment (start 119.405 105.41) (end 152.4 105.41) (width 0.25) (layer F.Cu) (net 15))
 (segment (start 166.624 91.186) (end 197.358 91.186) (width 0.25) (layer F.Cu) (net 15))
 (segment (start 152.4 105.41) (end 166.624 91.186) (width 0.25) (layer F.Cu) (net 15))
 (segment (start 118.965 107.13) (end 119.415 106.68) (width 0.25) (layer F.Cu) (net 17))
 (segment (start 117.715 107.13) (end 118.965 107.13) (width 0.25) (layer F.Cu) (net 17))
 (segment (start 119.415 106.68) (end 152.4 106.68) (width 0.25) (layer F.Cu) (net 17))
 (segment (start 199.034401 92.049599) (end 199.898 91.186) (width 0.25) (layer F.Cu) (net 17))
 (segment (start 198.709399 92.374601) (end 199.034401 92.049599) (width 0.25) (layer F.Cu) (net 17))
 (segment (start 166.705399 92.374601) (end 198.709399 92.374601) (width 0.25) (layer F.Cu) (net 17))
 (segment (start 152.4 106.68) (end 166.705399 92.374601) (width 0.25) (layer F.Cu) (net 17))
 (segment (start 118.115 100.65) (end 120.335 102.87) (width 0.25) (layer F.Cu) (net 11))
 (segment (start 117.715 100.65) (end 118.115 100.65) (width 0.25) (layer F.Cu) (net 11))
 (segment (start 120.335 102.87) (end 152.4 102.87) (width 0.25) (layer F.Cu) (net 11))
 (segment (start 166.624 88.646) (end 197.358 88.646) (width 0.25) (layer F.Cu) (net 11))
 (segment (start 152.4 102.87) (end 166.624 88.646) (width 0.25) (layer F.Cu) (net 11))
 (segment (start 199.034401 89.509599) (end 199.898 88.646) (width 0.25) (layer F.Cu) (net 13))
 (segment (start 117.715 102.81) (end 118.115 102.81) (width 0.25) (layer F.Cu) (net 13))
 (segment (start 118.115 102.81) (end 119.445 104.14) (width 0.25) (layer F.Cu) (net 13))
 (segment (start 119.445 104.14) (end 152.4 104.14) (width 0.25) (layer F.Cu) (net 13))
 (segment (start 152.4 104.14) (end 166.705399 89.834601) (width 0.25) (layer F.Cu) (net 13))
 (segment (start 166.705399 89.834601) (end 198.709399 89.834601) (width 0.25) (layer F.Cu) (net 13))
 (segment (start 198.709399 89.834601) (end 199.034401 89.509599) (width 0.25) (layer F.Cu) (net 13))
 (segment (start 136.144 86.106) (end 197.358 86.106) (width 0.25) (layer B.Cu) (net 16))
 (segment (start 118.51499 103.73501) (end 136.144 86.106) (width 0.25) (layer B.Cu) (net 16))
 (segment (start 115.05999 103.73501) (end 118.51499 103.73501) (width 0.25) (layer B.Cu) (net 16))
 (segment (start 113.425 104.97) (end 113.825 104.97) (width 0.25) (layer B.Cu) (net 16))
 (segment (start 113.825 104.97) (end 115.05999 103.73501) (width 0.25) (layer B.Cu) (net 16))
 (segment (start 115.90999 105.89501) (end 118.89499 105.89501) (width 0.25) (layer B.Cu) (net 18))
 (segment (start 113.425 107.13) (end 114.675 107.13) (width 0.25) (layer B.Cu) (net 18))
 (segment (start 114.675 107.13) (end 115.90999 105.89501) (width 0.25) (layer B.Cu) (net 18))
 (segment (start 118.89499 105.89501) (end 137.16 87.63) (width 0.25) (layer B.Cu) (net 18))
 (segment (start 199.034401 86.969599) (end 199.898 86.106) (width 0.25) (layer B.Cu) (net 18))
 (segment (start 198.709399 87.294601) (end 199.034401 86.969599) (width 0.25) (layer B.Cu) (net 18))
 (segment (start 173.055399 87.294601) (end 198.709399 87.294601) (width 0.25) (layer B.Cu) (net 18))
 (segment (start 172.72 87.63) (end 173.055399 87.294601) (width 0.25) (layer B.Cu) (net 18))
 (segment (start 137.16 87.63) (end 172.72 87.63) (width 0.25) (layer B.Cu) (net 18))
 (segment (start 115.90999 99.41501) (end 120.29499 99.41501) (width 0.25) (layer B.Cu) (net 12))
 (segment (start 113.425 100.65) (end 114.675 100.65) (width 0.25) (layer B.Cu) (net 12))
 (segment (start 114.675 100.65) (end 115.90999 99.41501) (width 0.25) (layer B.Cu) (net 12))
 (segment (start 136.144 83.566) (end 197.358 83.566) (width 0.25) (layer B.Cu) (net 12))
 (segment (start 120.29499 99.41501) (end 136.144 83.566) (width 0.25) (layer B.Cu) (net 12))
 (segment (start 115.081829 101.57501) (end 119.40499 101.57501) (width 0.25) (layer B.Cu) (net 14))
 (segment (start 113.425 102.81) (end 113.846839 102.81) (width 0.25) (layer B.Cu) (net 14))
 (segment (start 113.846839 102.81) (end 115.081829 101.57501) (width 0.25) (layer B.Cu) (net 14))
 (segment (start 199.034401 84.429599) (end 199.898 83.566) (width 0.25) (layer B.Cu) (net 14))
 (segment (start 198.709399 84.754601) (end 199.034401 84.429599) (width 0.25) (layer B.Cu) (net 14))
 (segment (start 136.225399 84.754601) (end 198.709399 84.754601) (width 0.25) (layer B.Cu) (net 14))
 (segment (start 119.40499 101.57501) (end 136.225399 84.754601) (width 0.25) (layer B.Cu) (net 14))
 (segment (start 118.115 98.49) (end 136.480389 80.124611) (width 0.25) (layer F.Cu) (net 9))
 (segment (start 117.715 98.49) (end 118.115 98.49) (width 0.25) (layer F.Cu) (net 9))
 (segment (start 196.456611 80.124611) (end 197.358 81.026) (width 0.25) (layer F.Cu) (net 9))
 (segment (start 136.480389 80.124611) (end 196.456611 80.124611) (width 0.25) (layer F.Cu) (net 9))
 (segment (start 118.115 94.17) (end 133.35 78.935) (width 0.25) (layer F.Cu) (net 7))
 (segment (start 117.715 94.17) (end 118.115 94.17) (width 0.25) (layer F.Cu) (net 7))
 (segment (start 196.136686 78.486) (end 197.358 78.486) (width 0.25) (layer F.Cu) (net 7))
 (segment (start 195.687686 78.935) (end 196.136686 78.486) (width 0.25) (layer F.Cu) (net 7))
 (segment (start 133.35 78.935) (end 195.687686 78.935) (width 0.25) (layer F.Cu) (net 7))
 (segment (start 199.034401 79.349599) (end 199.898 78.486) (width 0.25) (layer F.Cu) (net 8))
 (segment (start 198.709399 79.674601) (end 199.034401 79.349599) (width 0.25) (layer F.Cu) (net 8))
 (segment (start 134.770399 79.674601) (end 198.709399 79.674601) (width 0.25) (layer F.Cu) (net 8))
 (segment (start 118.115 96.33) (end 134.770399 79.674601) (width 0.25) (layer F.Cu) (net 8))
 (segment (start 117.715 96.33) (end 118.115 96.33) (width 0.25) (layer F.Cu) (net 8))
 (segment (start 118.115 89.85) (end 130.495 77.47) (width 0.25) (layer F.Cu) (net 5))
 (segment (start 117.715 89.85) (end 118.115 89.85) (width 0.25) (layer F.Cu) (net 5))
 (segment (start 195.834 77.47) (end 197.358 75.946) (width 0.25) (layer F.Cu) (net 5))
 (segment (start 130.495 77.47) (end 195.834 77.47) (width 0.25) (layer F.Cu) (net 5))
 (segment (start 118.115 92.01) (end 132.08 78.045) (width 0.25) (layer F.Cu) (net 6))
 (segment (start 117.715 92.01) (end 118.115 92.01) (width 0.25) (layer F.Cu) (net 6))
 (segment (start 199.034401 76.809599) (end 199.898 75.946) (width 0.25) (layer F.Cu) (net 6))
 (segment (start 198.709399 77.134601) (end 199.034401 76.809599) (width 0.25) (layer F.Cu) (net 6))
 (segment (start 196.805809 77.134601) (end 198.709399 77.134601) (width 0.25) (layer F.Cu) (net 6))
 (segment (start 195.89541 78.045) (end 196.805809 77.134601) (width 0.25) (layer F.Cu) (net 6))
 (segment (start 132.08 78.045) (end 195.89541 78.045) (width 0.25) (layer F.Cu) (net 6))
 (segment (start 118.965 85.53) (end 129.54 74.955) (width 0.25) (layer F.Cu) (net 3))
 (segment (start 117.715 85.53) (end 118.965 85.53) (width 0.25) (layer F.Cu) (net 3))
 (segment (start 195.809 74.955) (end 197.358 73.406) (width 0.25) (layer F.Cu) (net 3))
 (segment (start 129.54 74.955) (end 195.809 74.955) (width 0.25) (layer F.Cu) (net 3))
 (segment (start 117.715 87.69) (end 119.32 87.69) (width 0.25) (layer F.Cu) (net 4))
 (segment (start 118.115 87.69) (end 129.605 76.2) (width 0.25) (layer F.Cu) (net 4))
 (segment (start 117.715 87.69) (end 118.115 87.69) (width 0.25) (layer F.Cu) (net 4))
 (segment (start 199.034401 74.269599) (end 199.898 73.406) (width 0.25) (layer F.Cu) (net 4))
 (segment (start 198.709399 74.594601) (end 199.034401 74.269599) (width 0.25) (layer F.Cu) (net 4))
 (segment (start 196.805809 74.594601) (end 198.709399 74.594601) (width 0.25) (layer F.Cu) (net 4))
 (segment (start 195.20041 76.2) (end 196.805809 74.594601) (width 0.25) (layer F.Cu) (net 4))
 (segment (start 129.605 76.2) (end 195.20041 76.2) (width 0.25) (layer F.Cu) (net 4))
 (segment (start 186.757919 100.33) (end 187.96 100.33) (width 0.25) (layer F.Cu) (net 23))
 (segment (start 160.1216 100.33) (end 186.757919 100.33) (width 0.25) (layer F.Cu) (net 23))
 (segment (start 141.478 118.9736) (end 160.1216 100.33) (width 0.25) (layer F.Cu) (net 23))
 (segment (start 141.478 119.126) (end 141.478 118.9736) (width 0.25) (layer F.Cu) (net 23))
 (segment (start 200.761599 71.729599) (end 199.898 70.866) (width 0.25) (layer F.Cu) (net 23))
 (segment (start 201.086601 76.516529) (end 201.086601 72.054601) (width 0.25) (layer F.Cu) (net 23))
 (segment (start 200.66 76.94313) (end 201.086601 76.516529) (width 0.25) (layer F.Cu) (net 23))
 (segment (start 200.66 77.47) (end 200.66 76.94313) (width 0.25) (layer F.Cu) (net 23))
 (segment (start 201.086601 77.896601) (end 200.66 77.47) (width 0.25) (layer F.Cu) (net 23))
 (segment (start 200.66 82.02313) (end 201.086601 81.596529) (width 0.25) (layer F.Cu) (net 23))
 (segment (start 201.086601 81.596529) (end 201.086601 77.896601) (width 0.25) (layer F.Cu) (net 23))
 (segment (start 201.086601 82.976601) (end 200.66 82.55) (width 0.25) (layer F.Cu) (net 23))
 (segment (start 201.086601 86.676529) (end 201.086601 82.976601) (width 0.25) (layer F.Cu) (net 23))
 (segment (start 200.66 87.10313) (end 201.086601 86.676529) (width 0.25) (layer F.Cu) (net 23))
 (segment (start 200.66 87.63) (end 200.66 87.10313) (width 0.25) (layer F.Cu) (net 23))
 (segment (start 201.086601 88.056601) (end 200.66 87.63) (width 0.25) (layer F.Cu) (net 23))
 (segment (start 201.086601 99.376529) (end 201.086601 88.056601) (width 0.25) (layer F.Cu) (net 23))
 (segment (start 200.66 82.55) (end 200.66 82.02313) (width 0.25) (layer F.Cu) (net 23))
 (segment (start 200.468529 99.994601) (end 201.086601 99.376529) (width 0.25) (layer F.Cu) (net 23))
 (segment (start 201.086601 72.054601) (end 200.761599 71.729599) (width 0.25) (layer F.Cu) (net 23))
 (segment (start 189.49748 99.994601) (end 200.468529 99.994601) (width 0.25) (layer F.Cu) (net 23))
 (segment (start 189.162081 100.33) (end 189.49748 99.994601) (width 0.25) (layer F.Cu) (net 23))
 (segment (start 187.96 100.33) (end 189.162081 100.33) (width 0.25) (layer F.Cu) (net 23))
 (segment (start 199.898 70.866) (end 197.358 70.866) (width 0.25) (layer F.Cu) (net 23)))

